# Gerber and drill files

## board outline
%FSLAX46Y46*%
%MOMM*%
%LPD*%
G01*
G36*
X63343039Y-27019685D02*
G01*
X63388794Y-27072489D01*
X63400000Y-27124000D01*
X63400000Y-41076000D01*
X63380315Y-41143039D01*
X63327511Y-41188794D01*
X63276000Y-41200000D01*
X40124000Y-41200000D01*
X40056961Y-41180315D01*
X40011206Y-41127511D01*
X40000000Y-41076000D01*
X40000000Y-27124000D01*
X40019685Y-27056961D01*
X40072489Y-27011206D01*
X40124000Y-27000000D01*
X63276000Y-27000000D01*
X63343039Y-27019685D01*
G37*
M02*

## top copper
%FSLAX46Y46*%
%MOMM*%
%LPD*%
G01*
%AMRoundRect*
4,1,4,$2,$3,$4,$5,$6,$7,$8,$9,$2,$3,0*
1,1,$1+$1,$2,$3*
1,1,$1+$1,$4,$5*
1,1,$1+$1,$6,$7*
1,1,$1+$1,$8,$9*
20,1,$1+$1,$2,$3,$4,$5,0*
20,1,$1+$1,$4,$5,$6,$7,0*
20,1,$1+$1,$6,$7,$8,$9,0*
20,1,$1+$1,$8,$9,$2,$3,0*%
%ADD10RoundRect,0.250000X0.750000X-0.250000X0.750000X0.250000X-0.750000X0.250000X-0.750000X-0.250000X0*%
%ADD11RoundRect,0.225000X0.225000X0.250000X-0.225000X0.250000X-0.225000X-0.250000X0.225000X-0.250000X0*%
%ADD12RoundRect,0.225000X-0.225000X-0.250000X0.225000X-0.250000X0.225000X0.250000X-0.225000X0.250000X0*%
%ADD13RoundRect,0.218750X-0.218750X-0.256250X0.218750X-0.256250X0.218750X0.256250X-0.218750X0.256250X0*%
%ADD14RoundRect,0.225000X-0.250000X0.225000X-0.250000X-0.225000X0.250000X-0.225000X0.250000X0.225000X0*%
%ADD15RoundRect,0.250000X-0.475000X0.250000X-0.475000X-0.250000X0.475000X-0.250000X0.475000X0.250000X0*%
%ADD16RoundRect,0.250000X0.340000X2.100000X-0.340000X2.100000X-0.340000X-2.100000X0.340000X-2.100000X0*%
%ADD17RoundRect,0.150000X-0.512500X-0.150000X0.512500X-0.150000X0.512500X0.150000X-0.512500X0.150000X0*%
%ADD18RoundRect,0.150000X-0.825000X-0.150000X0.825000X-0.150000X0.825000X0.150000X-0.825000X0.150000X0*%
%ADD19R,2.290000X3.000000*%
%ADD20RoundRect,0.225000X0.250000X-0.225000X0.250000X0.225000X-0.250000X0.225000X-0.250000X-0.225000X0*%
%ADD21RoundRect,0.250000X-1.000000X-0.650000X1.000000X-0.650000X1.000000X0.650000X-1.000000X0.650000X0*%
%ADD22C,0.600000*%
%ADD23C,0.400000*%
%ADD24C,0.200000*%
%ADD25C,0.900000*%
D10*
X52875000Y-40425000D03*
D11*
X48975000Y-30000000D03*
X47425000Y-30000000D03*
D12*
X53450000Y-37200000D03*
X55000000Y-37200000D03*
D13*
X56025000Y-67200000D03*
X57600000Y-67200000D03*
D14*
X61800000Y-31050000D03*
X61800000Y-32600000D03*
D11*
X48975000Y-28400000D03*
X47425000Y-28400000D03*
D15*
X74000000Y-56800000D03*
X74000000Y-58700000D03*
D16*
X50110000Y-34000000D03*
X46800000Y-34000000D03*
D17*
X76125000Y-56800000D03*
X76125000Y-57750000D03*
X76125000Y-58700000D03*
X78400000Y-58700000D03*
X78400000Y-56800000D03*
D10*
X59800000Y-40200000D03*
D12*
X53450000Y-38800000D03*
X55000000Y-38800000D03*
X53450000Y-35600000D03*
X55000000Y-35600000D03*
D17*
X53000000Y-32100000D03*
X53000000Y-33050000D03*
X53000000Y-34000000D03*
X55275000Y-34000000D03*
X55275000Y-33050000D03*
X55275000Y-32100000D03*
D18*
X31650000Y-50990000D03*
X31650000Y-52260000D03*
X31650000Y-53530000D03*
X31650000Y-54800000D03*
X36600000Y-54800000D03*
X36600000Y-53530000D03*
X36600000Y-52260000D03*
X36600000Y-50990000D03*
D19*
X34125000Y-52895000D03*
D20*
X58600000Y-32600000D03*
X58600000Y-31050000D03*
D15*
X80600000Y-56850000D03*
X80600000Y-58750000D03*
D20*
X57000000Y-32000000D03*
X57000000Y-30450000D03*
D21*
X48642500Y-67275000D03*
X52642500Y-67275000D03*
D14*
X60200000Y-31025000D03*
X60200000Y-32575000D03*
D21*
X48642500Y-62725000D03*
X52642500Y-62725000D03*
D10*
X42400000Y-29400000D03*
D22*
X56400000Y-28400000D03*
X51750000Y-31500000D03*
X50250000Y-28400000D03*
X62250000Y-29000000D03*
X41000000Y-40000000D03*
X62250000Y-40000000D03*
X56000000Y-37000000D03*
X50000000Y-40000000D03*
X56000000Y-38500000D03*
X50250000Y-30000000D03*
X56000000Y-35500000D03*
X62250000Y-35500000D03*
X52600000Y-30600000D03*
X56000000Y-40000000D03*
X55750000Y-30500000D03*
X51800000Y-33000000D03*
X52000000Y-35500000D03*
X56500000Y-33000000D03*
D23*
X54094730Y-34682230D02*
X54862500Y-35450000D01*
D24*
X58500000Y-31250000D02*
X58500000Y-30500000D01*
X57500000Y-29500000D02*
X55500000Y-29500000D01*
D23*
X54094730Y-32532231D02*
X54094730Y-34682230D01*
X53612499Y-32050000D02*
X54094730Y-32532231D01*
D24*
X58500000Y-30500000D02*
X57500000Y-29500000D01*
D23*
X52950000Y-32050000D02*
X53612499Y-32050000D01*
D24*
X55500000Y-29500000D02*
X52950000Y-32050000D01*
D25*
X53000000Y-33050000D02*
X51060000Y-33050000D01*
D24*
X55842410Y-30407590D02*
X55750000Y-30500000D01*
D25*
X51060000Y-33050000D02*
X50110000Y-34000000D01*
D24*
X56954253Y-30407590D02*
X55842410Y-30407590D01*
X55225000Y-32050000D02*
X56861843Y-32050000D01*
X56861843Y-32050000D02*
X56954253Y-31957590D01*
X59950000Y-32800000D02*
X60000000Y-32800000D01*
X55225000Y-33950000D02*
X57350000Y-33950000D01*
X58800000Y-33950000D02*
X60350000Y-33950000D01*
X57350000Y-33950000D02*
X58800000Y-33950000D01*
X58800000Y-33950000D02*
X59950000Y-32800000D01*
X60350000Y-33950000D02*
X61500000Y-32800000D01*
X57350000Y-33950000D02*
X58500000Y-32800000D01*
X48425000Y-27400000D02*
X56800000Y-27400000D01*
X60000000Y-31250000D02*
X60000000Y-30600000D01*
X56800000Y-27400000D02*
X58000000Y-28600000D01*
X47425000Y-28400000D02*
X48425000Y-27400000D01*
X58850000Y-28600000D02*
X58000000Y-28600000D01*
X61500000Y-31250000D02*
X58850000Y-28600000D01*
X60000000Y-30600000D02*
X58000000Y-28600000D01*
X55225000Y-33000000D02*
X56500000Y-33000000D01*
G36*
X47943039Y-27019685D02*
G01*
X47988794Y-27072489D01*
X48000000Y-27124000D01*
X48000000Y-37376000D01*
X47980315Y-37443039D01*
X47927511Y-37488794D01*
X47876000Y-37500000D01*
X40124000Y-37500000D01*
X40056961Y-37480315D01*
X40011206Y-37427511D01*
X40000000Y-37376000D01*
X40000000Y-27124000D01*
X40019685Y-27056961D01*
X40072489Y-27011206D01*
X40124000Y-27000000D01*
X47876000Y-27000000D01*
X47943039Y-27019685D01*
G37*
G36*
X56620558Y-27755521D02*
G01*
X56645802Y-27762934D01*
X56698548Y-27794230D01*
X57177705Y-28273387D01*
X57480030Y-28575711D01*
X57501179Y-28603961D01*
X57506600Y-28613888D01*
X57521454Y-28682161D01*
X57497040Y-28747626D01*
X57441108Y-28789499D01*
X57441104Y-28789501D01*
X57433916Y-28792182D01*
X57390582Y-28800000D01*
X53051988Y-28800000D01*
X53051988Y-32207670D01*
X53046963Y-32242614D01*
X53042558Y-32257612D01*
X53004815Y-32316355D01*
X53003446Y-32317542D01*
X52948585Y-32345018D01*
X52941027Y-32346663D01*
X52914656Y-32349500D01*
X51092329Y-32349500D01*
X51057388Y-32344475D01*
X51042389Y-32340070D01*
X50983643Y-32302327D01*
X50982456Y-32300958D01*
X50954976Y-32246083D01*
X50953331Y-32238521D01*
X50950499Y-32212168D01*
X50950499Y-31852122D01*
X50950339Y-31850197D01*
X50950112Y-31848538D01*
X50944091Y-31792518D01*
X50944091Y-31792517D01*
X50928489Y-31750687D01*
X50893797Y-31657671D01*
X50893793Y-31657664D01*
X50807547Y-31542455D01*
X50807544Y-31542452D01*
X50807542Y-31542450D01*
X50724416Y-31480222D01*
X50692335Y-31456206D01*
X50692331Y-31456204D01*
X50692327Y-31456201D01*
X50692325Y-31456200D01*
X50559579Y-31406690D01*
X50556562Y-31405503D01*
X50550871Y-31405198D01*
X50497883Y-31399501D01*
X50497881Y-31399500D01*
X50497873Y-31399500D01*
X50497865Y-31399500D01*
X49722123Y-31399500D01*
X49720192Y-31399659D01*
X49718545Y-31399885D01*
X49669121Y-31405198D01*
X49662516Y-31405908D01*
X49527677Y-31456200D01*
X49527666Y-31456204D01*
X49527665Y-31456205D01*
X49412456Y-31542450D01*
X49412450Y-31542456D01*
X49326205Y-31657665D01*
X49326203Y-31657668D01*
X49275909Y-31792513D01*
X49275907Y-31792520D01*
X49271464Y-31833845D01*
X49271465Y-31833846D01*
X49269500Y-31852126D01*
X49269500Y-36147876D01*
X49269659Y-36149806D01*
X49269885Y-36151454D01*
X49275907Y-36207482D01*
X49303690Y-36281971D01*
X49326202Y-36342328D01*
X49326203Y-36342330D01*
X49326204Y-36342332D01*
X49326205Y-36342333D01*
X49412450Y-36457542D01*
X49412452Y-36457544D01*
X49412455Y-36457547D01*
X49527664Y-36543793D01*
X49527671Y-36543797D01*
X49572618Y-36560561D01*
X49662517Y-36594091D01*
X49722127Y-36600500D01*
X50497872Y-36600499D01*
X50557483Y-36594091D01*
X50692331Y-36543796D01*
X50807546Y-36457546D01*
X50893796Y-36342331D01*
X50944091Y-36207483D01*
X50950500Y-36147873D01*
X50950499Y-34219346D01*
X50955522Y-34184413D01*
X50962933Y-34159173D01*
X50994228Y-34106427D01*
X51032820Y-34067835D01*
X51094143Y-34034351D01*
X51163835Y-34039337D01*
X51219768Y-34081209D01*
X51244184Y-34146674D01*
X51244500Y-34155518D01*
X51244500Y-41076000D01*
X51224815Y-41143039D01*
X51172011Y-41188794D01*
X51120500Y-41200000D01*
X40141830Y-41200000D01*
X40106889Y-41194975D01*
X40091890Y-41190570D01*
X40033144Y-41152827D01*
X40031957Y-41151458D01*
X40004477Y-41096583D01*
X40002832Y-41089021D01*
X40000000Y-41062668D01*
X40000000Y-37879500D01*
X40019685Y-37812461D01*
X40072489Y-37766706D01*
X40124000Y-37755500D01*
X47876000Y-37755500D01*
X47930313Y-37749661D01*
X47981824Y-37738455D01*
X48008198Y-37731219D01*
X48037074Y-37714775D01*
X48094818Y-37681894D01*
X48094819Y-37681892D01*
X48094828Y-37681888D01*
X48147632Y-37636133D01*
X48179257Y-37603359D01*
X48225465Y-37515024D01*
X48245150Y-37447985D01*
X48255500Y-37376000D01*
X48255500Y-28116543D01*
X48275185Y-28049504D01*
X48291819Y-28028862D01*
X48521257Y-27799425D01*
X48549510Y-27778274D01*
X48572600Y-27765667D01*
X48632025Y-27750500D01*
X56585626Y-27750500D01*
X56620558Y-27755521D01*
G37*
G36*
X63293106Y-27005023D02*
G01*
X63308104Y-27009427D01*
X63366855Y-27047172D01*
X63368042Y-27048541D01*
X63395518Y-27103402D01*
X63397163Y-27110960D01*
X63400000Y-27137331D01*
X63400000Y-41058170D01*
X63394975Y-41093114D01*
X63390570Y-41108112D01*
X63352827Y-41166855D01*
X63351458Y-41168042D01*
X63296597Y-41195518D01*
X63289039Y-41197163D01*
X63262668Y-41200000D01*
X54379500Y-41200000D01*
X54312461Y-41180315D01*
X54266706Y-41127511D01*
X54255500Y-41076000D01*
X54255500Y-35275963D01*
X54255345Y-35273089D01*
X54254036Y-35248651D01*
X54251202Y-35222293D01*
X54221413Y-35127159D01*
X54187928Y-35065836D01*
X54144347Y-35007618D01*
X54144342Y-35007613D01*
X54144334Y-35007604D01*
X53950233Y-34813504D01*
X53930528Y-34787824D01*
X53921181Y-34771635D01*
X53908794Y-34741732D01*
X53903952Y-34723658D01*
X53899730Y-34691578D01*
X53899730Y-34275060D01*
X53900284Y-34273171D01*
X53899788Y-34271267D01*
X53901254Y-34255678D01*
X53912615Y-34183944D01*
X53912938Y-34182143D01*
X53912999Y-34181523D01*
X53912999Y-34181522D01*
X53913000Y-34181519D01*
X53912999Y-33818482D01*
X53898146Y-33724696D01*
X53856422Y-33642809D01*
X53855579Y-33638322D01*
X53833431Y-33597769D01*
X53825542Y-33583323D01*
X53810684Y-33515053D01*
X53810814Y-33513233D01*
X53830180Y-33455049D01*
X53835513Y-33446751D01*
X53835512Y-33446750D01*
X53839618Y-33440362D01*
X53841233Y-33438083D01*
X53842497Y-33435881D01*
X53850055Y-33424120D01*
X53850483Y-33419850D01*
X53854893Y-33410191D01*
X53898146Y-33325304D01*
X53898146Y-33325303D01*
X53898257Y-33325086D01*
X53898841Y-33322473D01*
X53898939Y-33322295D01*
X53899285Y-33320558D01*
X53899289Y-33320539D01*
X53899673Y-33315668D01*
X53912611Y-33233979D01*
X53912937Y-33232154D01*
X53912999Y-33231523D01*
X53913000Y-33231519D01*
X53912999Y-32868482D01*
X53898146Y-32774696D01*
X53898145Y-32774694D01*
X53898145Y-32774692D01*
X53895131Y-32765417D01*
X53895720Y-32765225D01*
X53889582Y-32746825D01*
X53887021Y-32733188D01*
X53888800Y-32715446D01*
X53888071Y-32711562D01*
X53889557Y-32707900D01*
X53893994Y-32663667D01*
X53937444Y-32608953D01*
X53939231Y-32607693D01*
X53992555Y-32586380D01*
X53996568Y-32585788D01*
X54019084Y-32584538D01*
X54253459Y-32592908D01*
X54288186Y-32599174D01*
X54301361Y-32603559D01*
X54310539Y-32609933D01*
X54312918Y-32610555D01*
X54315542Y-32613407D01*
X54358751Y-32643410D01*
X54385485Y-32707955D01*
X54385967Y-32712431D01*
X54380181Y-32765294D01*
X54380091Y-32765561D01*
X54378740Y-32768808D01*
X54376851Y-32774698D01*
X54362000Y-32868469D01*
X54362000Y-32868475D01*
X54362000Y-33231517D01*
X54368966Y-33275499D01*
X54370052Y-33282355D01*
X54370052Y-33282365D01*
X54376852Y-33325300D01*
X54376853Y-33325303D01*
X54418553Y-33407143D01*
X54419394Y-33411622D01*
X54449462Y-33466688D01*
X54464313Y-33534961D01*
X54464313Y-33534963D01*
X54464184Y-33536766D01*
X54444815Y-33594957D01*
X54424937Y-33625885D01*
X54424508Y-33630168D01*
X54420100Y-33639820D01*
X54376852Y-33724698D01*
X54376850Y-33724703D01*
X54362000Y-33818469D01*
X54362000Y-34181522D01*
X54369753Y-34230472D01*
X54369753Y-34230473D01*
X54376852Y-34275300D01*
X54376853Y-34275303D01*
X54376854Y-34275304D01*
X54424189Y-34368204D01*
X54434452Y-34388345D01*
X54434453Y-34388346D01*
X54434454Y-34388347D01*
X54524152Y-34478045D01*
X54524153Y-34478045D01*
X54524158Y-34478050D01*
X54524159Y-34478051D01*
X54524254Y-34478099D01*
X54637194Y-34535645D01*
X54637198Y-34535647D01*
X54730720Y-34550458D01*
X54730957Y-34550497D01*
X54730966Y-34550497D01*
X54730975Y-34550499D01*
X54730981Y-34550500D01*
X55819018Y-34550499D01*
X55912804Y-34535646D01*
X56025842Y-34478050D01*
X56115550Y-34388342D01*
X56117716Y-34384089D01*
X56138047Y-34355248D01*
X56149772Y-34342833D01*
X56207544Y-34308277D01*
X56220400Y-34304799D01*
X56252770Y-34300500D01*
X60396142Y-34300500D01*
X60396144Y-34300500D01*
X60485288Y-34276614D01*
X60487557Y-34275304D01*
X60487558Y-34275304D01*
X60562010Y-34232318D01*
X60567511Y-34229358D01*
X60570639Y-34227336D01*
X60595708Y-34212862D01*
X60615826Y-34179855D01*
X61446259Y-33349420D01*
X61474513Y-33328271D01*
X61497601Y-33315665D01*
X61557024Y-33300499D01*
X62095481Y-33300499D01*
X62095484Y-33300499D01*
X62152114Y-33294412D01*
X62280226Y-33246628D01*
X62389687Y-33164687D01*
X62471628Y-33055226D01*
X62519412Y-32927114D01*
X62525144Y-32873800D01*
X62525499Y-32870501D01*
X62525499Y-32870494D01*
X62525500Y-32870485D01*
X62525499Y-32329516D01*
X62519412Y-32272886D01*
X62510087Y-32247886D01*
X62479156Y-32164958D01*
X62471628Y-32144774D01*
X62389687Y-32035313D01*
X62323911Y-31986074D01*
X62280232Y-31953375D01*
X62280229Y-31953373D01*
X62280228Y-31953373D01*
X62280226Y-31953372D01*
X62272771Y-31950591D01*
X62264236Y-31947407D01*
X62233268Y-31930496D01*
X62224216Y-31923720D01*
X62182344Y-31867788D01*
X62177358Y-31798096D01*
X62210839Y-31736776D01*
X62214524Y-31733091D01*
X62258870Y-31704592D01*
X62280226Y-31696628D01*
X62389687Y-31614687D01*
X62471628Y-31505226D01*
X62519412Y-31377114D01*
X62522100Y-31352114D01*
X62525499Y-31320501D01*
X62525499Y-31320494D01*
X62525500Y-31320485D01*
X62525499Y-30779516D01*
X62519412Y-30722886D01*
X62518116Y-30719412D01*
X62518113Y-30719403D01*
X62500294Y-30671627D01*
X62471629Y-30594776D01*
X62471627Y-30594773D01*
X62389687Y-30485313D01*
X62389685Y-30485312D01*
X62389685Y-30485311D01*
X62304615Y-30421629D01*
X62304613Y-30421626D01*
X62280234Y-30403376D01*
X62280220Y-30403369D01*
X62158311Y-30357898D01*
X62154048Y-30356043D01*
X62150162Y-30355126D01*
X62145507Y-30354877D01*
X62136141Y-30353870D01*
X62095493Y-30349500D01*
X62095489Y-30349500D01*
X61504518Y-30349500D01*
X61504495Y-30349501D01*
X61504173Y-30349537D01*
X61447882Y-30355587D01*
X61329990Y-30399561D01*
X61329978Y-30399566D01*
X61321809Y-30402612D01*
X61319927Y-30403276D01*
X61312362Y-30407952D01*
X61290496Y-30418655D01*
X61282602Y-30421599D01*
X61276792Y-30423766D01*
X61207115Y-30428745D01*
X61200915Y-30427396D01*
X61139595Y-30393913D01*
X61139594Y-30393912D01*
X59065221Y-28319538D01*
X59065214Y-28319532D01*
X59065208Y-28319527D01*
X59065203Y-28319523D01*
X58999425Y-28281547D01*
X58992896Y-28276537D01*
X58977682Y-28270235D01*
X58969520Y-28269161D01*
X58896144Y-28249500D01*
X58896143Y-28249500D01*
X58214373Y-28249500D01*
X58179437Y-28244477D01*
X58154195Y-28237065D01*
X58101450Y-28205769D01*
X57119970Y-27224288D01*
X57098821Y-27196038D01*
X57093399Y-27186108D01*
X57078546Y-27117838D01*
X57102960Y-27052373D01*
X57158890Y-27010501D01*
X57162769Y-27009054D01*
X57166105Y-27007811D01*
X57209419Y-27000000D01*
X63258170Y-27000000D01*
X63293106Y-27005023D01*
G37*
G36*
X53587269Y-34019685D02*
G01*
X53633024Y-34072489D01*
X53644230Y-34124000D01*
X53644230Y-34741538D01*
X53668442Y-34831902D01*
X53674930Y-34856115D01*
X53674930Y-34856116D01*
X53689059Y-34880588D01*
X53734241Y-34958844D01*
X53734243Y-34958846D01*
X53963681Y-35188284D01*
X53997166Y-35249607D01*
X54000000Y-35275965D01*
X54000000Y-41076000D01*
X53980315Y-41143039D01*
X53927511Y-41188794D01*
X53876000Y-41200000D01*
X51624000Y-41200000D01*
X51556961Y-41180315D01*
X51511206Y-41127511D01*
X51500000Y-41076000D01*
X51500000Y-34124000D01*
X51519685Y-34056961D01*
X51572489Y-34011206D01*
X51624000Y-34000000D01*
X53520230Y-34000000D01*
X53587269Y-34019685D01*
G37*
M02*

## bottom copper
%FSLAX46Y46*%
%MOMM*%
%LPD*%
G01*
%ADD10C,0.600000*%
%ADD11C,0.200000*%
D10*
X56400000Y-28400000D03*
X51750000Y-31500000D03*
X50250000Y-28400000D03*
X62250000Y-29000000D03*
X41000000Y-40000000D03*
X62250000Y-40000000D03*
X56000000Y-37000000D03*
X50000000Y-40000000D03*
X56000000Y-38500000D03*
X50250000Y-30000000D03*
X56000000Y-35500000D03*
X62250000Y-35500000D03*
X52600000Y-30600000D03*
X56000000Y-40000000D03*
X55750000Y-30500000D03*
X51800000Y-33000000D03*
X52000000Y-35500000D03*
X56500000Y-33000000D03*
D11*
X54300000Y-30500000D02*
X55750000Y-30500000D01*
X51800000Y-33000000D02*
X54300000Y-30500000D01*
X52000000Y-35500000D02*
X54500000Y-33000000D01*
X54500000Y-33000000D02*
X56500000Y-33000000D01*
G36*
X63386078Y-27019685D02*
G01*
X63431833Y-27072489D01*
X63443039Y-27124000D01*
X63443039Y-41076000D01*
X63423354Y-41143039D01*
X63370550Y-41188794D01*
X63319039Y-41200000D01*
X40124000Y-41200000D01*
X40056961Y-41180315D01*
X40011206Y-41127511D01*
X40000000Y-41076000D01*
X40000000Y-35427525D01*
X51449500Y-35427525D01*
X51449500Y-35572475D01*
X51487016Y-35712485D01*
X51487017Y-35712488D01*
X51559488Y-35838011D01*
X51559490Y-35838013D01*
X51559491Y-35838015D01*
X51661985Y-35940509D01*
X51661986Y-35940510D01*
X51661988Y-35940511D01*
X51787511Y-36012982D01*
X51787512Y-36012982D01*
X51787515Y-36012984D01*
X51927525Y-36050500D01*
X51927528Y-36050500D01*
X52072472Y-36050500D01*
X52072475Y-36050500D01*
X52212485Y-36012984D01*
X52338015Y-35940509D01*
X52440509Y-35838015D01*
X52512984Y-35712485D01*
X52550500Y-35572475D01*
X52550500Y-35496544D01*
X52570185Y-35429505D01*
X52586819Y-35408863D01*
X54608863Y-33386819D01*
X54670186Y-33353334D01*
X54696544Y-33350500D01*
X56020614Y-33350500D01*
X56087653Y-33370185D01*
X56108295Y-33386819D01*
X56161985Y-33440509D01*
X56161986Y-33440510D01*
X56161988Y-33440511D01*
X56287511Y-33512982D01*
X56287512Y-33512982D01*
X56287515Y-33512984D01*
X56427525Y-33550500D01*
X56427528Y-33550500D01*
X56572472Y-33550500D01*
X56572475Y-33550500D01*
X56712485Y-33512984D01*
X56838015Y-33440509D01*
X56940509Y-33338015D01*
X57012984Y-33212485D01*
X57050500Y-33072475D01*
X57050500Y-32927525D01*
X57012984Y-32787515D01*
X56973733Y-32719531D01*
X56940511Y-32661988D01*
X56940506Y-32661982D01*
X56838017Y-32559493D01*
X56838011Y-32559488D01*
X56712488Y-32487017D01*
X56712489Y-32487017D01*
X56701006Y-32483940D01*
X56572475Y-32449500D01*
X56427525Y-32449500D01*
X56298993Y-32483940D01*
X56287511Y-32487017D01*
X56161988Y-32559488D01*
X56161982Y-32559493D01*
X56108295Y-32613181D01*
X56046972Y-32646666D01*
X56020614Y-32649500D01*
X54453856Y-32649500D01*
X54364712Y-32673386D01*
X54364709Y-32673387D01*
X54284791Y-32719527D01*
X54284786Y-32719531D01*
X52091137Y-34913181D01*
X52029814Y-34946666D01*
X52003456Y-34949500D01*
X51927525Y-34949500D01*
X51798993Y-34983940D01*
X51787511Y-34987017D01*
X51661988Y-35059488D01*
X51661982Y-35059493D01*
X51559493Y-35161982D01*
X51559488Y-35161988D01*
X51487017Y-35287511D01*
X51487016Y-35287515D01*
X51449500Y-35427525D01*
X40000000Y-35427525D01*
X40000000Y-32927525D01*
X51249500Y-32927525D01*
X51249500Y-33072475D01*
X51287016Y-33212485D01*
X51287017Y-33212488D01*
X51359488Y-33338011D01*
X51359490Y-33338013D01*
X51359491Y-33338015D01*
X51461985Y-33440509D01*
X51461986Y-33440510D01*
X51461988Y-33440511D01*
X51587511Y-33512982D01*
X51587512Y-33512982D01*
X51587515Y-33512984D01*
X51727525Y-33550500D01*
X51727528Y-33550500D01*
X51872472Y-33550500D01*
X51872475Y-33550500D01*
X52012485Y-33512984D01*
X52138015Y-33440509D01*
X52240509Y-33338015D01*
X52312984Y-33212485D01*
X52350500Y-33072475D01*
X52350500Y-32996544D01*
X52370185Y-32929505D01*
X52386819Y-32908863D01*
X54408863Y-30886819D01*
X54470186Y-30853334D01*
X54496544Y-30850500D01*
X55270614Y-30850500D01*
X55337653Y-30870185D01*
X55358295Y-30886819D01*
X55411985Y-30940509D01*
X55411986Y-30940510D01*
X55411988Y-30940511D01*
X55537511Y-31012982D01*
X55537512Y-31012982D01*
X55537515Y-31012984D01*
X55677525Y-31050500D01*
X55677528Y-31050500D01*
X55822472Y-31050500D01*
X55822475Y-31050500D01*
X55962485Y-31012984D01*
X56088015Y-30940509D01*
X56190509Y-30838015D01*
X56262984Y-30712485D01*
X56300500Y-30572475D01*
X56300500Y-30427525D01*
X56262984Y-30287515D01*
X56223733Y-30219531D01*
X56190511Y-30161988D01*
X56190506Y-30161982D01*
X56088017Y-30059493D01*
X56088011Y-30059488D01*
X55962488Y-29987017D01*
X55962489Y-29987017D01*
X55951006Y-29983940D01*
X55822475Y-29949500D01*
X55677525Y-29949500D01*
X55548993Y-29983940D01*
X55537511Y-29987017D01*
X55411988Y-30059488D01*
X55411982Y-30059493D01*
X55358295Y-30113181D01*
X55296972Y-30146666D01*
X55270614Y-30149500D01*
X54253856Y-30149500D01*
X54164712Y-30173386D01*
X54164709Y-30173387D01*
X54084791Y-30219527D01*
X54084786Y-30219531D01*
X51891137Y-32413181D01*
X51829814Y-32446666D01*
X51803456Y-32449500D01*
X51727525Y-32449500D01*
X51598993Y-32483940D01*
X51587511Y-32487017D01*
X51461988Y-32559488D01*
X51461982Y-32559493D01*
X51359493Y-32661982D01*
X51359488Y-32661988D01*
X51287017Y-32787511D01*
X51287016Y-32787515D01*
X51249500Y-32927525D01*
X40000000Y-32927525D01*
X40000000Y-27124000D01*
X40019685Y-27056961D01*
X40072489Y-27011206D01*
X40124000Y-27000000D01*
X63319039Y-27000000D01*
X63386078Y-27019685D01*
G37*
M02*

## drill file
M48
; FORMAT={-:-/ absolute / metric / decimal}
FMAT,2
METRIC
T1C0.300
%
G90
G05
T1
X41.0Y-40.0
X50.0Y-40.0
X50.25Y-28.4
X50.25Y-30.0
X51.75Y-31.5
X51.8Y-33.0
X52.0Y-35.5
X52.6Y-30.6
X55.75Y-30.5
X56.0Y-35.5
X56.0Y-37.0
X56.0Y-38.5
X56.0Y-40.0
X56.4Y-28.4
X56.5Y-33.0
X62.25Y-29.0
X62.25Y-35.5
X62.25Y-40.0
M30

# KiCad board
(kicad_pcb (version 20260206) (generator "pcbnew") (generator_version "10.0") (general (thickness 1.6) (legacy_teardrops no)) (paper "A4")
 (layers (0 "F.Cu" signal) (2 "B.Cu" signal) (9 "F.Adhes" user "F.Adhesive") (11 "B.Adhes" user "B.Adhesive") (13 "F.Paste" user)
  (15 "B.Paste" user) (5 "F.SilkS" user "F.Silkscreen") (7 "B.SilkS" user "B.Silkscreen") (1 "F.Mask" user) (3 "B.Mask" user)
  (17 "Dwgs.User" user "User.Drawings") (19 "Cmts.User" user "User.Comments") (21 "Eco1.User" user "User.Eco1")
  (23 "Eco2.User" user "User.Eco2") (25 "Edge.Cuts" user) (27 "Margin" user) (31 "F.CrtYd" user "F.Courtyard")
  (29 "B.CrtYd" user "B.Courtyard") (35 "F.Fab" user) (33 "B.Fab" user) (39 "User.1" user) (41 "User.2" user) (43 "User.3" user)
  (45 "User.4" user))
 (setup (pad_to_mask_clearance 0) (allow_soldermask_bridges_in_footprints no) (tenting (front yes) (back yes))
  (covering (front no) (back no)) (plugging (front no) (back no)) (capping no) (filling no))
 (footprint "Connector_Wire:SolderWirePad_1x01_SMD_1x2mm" (layer "F.Cu") (at 52.875 40.425 90)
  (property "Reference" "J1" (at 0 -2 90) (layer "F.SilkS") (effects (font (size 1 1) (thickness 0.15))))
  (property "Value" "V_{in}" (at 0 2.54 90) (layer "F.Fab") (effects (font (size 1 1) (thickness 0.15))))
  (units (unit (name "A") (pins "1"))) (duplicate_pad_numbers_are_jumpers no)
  (pad "1" smd roundrect (at 0 0 90) (size 1 2) (layers "F.Cu" "F.Mask") (roundrect_rratio 0.25) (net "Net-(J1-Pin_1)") (zone_connect 2)))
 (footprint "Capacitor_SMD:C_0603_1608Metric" (layer "F.Cu") (at 48.2 30 180)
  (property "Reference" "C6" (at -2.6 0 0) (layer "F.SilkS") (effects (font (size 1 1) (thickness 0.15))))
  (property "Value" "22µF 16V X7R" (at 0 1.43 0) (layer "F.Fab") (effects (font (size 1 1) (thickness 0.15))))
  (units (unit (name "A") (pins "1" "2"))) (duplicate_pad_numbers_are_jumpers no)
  (pad "1" smd roundrect (at -0.775 0 180) (size 0.9 0.95) (layers "F.Cu" "F.Mask" "F.Paste") (roundrect_rratio 0.25) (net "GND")
   (zone_connect 2))
  (pad "2" smd roundrect (at 0.775 0 180) (size 0.9 0.95) (layers "F.Cu" "F.Mask" "F.Paste") (roundrect_rratio 0.25) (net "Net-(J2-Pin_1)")
   (zone_connect 2)))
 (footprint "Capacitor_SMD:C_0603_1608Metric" (layer "F.Cu") (at 54.225 37.2)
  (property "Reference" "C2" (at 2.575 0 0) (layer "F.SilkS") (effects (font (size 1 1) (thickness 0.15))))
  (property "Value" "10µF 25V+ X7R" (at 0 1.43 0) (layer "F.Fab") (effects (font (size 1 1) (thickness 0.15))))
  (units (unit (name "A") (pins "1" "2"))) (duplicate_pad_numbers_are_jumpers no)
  (pad "1" smd roundrect (at -0.775 0) (size 0.9 0.95) (layers "F.Cu" "F.Mask" "F.Paste") (roundrect_rratio 0.25) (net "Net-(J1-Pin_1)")
   (zone_connect 2))
  (pad "2" smd roundrect (at 0.775 0) (size 0.9 0.95) (layers "F.Cu" "F.Mask" "F.Paste") (roundrect_rratio 0.25) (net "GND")
   (zone_connect 2)))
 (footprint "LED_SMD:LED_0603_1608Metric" (layer "F.Cu") (at 56.8125 67.2)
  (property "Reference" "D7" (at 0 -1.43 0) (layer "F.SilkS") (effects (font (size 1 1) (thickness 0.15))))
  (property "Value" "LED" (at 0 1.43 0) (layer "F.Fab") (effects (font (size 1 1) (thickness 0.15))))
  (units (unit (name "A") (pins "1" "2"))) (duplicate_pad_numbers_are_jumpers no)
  (pad "1" smd roundrect (at -0.7875 0) (size 0.875 0.95) (layers "F.Cu" "F.Mask" "F.Paste") (roundrect_rratio 0.25) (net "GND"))
  (pad "2" smd roundrect (at 0.7875 0) (size 0.875 0.95) (layers "F.Cu" "F.Mask" "F.Paste") (roundrect_rratio 0.25) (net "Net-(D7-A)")))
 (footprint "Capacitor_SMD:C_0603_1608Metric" (layer "F.Cu") (at 61.8 31.825 -90)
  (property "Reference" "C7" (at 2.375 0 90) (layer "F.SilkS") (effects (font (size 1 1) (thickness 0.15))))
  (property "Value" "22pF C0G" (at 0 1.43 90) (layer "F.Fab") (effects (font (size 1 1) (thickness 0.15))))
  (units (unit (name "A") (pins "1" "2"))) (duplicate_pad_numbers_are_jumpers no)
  (pad "1" smd roundrect (at -0.775 0 270) (size 0.9 0.95) (layers "F.Cu" "F.Mask" "F.Paste") (roundrect_rratio 0.25) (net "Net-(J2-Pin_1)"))
  (pad "2" smd roundrect (at 0.775 0 270) (size 0.9 0.95) (layers "F.Cu" "F.Mask" "F.Paste") (roundrect_rratio 0.25) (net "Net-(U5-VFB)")))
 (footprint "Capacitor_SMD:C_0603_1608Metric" (layer "F.Cu") (at 48.2 28.4 180)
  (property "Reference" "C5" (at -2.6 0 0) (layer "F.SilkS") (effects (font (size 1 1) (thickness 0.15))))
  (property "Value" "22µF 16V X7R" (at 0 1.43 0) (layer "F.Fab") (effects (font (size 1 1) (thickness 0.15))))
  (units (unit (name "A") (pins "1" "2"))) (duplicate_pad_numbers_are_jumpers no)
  (pad "1" smd roundrect (at -0.775 0 180) (size 0.9 0.95) (layers "F.Cu" "F.Mask" "F.Paste") (roundrect_rratio 0.25) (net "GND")
   (zone_connect 2))
  (pad "2" smd roundrect (at 0.775 0 180) (size 0.9 0.95) (layers "F.Cu" "F.Mask" "F.Paste") (roundrect_rratio 0.25) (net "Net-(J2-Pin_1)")
   (zone_connect 2)))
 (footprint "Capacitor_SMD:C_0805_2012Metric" (layer "F.Cu") (at 74 57.75 -90)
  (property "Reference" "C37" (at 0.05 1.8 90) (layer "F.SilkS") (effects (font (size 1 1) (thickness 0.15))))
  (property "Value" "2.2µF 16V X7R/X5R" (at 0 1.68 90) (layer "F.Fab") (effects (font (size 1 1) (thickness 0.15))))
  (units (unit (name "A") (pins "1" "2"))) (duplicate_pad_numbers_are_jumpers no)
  (pad "1" smd roundrect (at -0.95 0 270) (size 1 1.45) (layers "F.Cu" "F.Mask" "F.Paste") (roundrect_rratio 0.25) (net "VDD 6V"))
  (pad "2" smd roundrect (at 0.95 0 270) (size 1 1.45) (layers "F.Cu" "F.Mask" "F.Paste") (roundrect_rratio 0.25) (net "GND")))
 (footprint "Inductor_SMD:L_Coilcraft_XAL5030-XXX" (layer "F.Cu") (at 48.455 34 180)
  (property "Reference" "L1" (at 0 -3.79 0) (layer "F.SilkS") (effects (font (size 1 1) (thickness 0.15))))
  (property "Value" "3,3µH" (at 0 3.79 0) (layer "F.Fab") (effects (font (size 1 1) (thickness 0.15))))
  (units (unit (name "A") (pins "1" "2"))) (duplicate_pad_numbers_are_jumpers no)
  (pad "1" smd roundrect (at -1.655 0 180) (size 1.18 4.7) (layers "F.Cu" "F.Mask" "F.Paste") (roundrect_rratio 0.211864)
   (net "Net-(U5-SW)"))
  (pad "2" smd roundrect (at 1.655 0 180) (size 1.18 4.7) (layers "F.Cu" "F.Mask" "F.Paste") (roundrect_rratio 0.211864)
   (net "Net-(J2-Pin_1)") (zone_connect 2)))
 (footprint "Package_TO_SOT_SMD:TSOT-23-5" (layer "F.Cu") (at 77.2625 57.75)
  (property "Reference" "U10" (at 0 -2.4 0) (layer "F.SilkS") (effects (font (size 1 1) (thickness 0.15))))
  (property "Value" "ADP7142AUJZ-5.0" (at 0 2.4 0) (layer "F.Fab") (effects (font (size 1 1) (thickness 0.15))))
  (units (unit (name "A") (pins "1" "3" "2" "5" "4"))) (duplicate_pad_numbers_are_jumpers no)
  (pad "1" smd roundrect (at -1.1375 -0.95) (size 1.325 0.6) (layers "F.Cu" "F.Mask" "F.Paste") (roundrect_rratio 0.25) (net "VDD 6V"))
  (pad "2" smd roundrect (at -1.1375 0) (size 1.325 0.6) (layers "F.Cu" "F.Mask" "F.Paste") (roundrect_rratio 0.25) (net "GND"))
  (pad "3" smd roundrect (at -1.1375 0.95) (size 1.325 0.6) (layers "F.Cu" "F.Mask" "F.Paste") (roundrect_rratio 0.25) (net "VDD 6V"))
  (pad "4" smd roundrect (at 1.1375 0.95) (size 1.325 0.6) (layers "F.Cu" "F.Mask" "F.Paste") (roundrect_rratio 0.25) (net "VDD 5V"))
  (pad "5" smd roundrect (at 1.1375 -0.95) (size 1.325 0.6) (layers "F.Cu" "F.Mask" "F.Paste") (roundrect_rratio 0.25) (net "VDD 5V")))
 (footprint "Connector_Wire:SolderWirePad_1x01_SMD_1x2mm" (layer "F.Cu") (at 59.8 40.2 90)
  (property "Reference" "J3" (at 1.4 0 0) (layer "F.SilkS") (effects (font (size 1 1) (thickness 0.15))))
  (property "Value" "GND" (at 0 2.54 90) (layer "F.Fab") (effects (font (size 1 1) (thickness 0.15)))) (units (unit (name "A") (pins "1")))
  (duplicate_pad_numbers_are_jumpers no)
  (pad "1" smd roundrect (at 0 0 90) (size 1 2) (layers "F.Cu" "F.Mask") (roundrect_rratio 0.25) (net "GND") (zone_connect 2)))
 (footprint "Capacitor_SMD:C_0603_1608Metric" (layer "F.Cu") (at 54.225 38.8)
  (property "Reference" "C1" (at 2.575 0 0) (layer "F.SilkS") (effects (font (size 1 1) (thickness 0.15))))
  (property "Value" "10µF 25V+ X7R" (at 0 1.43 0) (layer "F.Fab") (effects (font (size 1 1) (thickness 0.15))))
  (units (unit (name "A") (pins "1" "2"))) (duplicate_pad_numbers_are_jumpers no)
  (pad "1" smd roundrect (at -0.775 0) (size 0.9 0.95) (layers "F.Cu" "F.Mask" "F.Paste") (roundrect_rratio 0.25) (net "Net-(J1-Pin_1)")
   (zone_connect 2))
  (pad "2" smd roundrect (at 0.775 0) (size 0.9 0.95) (layers "F.Cu" "F.Mask" "F.Paste") (roundrect_rratio 0.25) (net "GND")
   (zone_connect 2)))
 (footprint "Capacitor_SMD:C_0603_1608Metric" (layer "F.Cu") (at 54.225 35.6)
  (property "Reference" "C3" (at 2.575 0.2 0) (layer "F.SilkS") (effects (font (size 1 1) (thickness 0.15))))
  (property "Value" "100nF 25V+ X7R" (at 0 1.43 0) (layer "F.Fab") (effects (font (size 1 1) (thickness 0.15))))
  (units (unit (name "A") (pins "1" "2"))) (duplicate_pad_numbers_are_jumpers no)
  (pad "1" smd roundrect (at -0.775 0) (size 0.9 0.95) (layers "F.Cu" "F.Mask" "F.Paste") (roundrect_rratio 0.25) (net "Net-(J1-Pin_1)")
   (zone_connect 2))
  (pad "2" smd roundrect (at 0.775 0) (size 0.9 0.95) (layers "F.Cu" "F.Mask" "F.Paste") (roundrect_rratio 0.25) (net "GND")
   (zone_connect 2)))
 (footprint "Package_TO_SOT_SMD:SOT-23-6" (layer "F.Cu") (at 54.1375 33.05)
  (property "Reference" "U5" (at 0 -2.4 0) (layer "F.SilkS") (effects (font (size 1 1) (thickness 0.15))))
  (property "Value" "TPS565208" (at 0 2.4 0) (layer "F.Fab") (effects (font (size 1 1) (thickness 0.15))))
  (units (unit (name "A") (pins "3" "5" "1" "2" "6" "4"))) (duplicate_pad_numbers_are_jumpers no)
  (pad "1" smd roundrect (at -1.1375 -0.95) (size 1.325 0.6) (layers "F.Cu" "F.Mask" "F.Paste") (roundrect_rratio 0.25) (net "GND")
   (zone_connect 2))
  (pad "2" smd roundrect (at -1.1375 0) (size 1.325 0.6) (layers "F.Cu" "F.Mask" "F.Paste") (roundrect_rratio 0.25) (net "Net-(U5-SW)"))
  (pad "3" smd roundrect (at -1.1375 0.95) (size 1.325 0.6) (layers "F.Cu" "F.Mask" "F.Paste") (roundrect_rratio 0.25)
   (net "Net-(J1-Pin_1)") (zone_connect 2))
  (pad "4" smd roundrect (at 1.1375 0.95) (size 1.325 0.6) (layers "F.Cu" "F.Mask" "F.Paste") (roundrect_rratio 0.25) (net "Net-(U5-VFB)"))
  (pad "5" smd roundrect (at 1.1375 0) (size 1.325 0.6) (layers "F.Cu" "F.Mask" "F.Paste") (roundrect_rratio 0.25) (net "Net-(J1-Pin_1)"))
  (pad "6" smd roundrect (at 1.1375 -0.95) (size 1.325 0.6) (layers "F.Cu" "F.Mask" "F.Paste") (roundrect_rratio 0.25) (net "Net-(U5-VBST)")))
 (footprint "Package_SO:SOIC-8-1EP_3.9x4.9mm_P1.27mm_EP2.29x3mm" (layer "F.Cu") (at 34.125 52.895)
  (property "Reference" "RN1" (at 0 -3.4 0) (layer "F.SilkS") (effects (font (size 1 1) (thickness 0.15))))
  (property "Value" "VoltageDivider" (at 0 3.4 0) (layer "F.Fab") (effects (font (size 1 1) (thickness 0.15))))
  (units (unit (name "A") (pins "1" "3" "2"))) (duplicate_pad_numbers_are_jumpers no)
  (pad "" smd roundrect (at -0.57 -0.75) (size 0.92 1.21) (layers "F.Paste") (roundrect_rratio 0.25))
  (pad "" smd roundrect (at -0.57 0.75) (size 0.92 1.21) (layers "F.Paste") (roundrect_rratio 0.25))
  (pad "" smd roundrect (at 0.57 -0.75) (size 0.92 1.21) (layers "F.Paste") (roundrect_rratio 0.25))
  (pad "" smd roundrect (at 0.57 0.75) (size 0.92 1.21) (layers "F.Paste") (roundrect_rratio 0.25))
  (pad "1" smd roundrect (at -2.475 -1.905) (size 1.95 0.6) (layers "F.Cu" "F.Mask" "F.Paste") (roundrect_rratio 0.25) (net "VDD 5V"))
  (pad "2" smd roundrect (at -2.475 -0.635) (size 1.95 0.6) (layers "F.Cu" "F.Mask" "F.Paste") (roundrect_rratio 0.25) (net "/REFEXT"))
  (pad "3" smd roundrect (at -2.475 0.635) (size 1.95 0.6) (layers "F.Cu" "F.Mask" "F.Paste") (roundrect_rratio 0.25) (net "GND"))
  (pad "4" smd roundrect (at -2.475 1.905) (size 1.95 0.6) (layers "F.Cu" "F.Mask" "F.Paste") (roundrect_rratio 0.25))
  (pad "5" smd roundrect (at 2.475 1.905) (size 1.95 0.6) (layers "F.Cu" "F.Mask" "F.Paste") (roundrect_rratio 0.25))
  (pad "6" smd roundrect (at 2.475 0.635) (size 1.95 0.6) (layers "F.Cu" "F.Mask" "F.Paste") (roundrect_rratio 0.25))
  (pad "7" smd roundrect (at 2.475 -0.635) (size 1.95 0.6) (layers "F.Cu" "F.Mask" "F.Paste") (roundrect_rratio 0.25))
  (pad "8" smd roundrect (at 2.475 -1.905) (size 1.95 0.6) (layers "F.Cu" "F.Mask" "F.Paste") (roundrect_rratio 0.25))
  (pad "9" smd rect (at 0 0) (size 2.29 3) (layers "F.Cu" "F.Mask") (zone_connect 2)))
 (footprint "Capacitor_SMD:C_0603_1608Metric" (layer "F.Cu") (at 58.6 31.825 90)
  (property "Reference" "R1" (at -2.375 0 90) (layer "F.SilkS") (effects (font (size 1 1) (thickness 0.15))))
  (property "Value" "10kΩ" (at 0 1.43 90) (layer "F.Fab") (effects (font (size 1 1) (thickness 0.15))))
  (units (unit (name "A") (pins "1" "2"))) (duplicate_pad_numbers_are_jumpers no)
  (pad "1" smd roundrect (at -0.775 0 90) (size 0.9 0.95) (layers "F.Cu" "F.Mask" "F.Paste") (roundrect_rratio 0.25) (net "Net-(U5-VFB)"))
  (pad "2" smd roundrect (at 0.775 0 90) (size 0.9 0.95) (layers "F.Cu" "F.Mask" "F.Paste") (roundrect_rratio 0.25) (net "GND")))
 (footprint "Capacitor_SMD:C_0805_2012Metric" (layer "F.Cu") (at 80.6 57.8 -90)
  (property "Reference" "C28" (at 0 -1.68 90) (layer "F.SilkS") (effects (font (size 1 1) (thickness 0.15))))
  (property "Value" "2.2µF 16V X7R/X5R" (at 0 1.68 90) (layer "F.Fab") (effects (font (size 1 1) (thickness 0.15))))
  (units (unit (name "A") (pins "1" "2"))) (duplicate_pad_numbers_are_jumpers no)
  (pad "1" smd roundrect (at -0.95 0 270) (size 1 1.45) (layers "F.Cu" "F.Mask" "F.Paste") (roundrect_rratio 0.25) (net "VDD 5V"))
  (pad "2" smd roundrect (at 0.95 0 270) (size 1 1.45) (layers "F.Cu" "F.Mask" "F.Paste") (roundrect_rratio 0.25) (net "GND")))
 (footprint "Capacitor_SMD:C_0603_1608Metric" (layer "F.Cu") (at 57 31.225 90)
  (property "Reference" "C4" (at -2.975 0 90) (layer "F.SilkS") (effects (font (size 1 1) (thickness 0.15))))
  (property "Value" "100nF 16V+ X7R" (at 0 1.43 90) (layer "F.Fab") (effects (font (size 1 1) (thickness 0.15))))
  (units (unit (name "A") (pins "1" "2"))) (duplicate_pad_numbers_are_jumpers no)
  (pad "1" smd roundrect (at -0.775 0 90) (size 0.9 0.95) (layers "F.Cu" "F.Mask" "F.Paste") (roundrect_rratio 0.25) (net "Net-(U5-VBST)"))
  (pad "2" smd roundrect (at 0.775 0 90) (size 0.9 0.95) (layers "F.Cu" "F.Mask" "F.Paste") (roundrect_rratio 0.25) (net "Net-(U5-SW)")))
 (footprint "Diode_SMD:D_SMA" (layer "F.Cu") (at 50.6425 67.275)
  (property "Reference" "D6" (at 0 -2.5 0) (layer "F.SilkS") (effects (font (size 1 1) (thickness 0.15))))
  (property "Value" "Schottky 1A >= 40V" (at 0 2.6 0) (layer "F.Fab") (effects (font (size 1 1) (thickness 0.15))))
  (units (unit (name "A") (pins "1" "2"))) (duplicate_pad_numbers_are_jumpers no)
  (pad "1" smd roundrect (at -2 0) (size 2.5 1.8) (layers "F.Cu" "F.Mask" "F.Paste") (roundrect_rratio 0.1388888889) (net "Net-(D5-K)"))
  (pad "2" smd roundrect (at 2 0) (size 2.5 1.8) (layers "F.Cu" "F.Mask" "F.Paste") (roundrect_rratio 0.1388888889) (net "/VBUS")))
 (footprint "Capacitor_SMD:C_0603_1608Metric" (layer "F.Cu") (at 60.2 31.8 -90)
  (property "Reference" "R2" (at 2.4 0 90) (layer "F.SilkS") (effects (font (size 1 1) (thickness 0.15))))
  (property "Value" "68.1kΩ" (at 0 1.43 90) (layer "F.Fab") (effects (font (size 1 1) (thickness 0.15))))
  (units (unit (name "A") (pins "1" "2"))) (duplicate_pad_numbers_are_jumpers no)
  (pad "1" smd roundrect (at -0.775 0 270) (size 0.9 0.95) (layers "F.Cu" "F.Mask" "F.Paste") (roundrect_rratio 0.25) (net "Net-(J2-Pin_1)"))
  (pad "2" smd roundrect (at 0.775 0 270) (size 0.9 0.95) (layers "F.Cu" "F.Mask" "F.Paste") (roundrect_rratio 0.25) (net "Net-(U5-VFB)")))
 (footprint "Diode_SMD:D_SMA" (layer "F.Cu") (at 50.6425 62.725)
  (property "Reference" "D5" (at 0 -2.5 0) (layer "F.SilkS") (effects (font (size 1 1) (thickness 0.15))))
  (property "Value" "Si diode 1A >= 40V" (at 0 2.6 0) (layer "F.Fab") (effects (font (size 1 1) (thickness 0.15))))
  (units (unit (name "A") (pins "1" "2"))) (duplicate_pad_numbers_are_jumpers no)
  (pad "1" smd roundrect (at -2 0) (size 2.5 1.8) (layers "F.Cu" "F.Mask" "F.Paste") (roundrect_rratio 0.1388888889) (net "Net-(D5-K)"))
  (pad "2" smd roundrect (at 2 0) (size 2.5 1.8) (layers "F.Cu" "F.Mask" "F.Paste") (roundrect_rratio 0.1388888889) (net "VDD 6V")))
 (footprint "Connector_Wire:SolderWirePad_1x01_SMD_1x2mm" (layer "F.Cu") (at 42.4 29.4 90)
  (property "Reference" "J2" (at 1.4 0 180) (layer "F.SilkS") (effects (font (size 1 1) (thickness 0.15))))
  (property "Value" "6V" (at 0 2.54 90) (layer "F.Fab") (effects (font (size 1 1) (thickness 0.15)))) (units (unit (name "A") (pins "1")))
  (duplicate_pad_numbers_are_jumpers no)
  (pad "1" smd roundrect (at 0 0 90) (size 1 2) (layers "F.Cu" "F.Mask") (roundrect_rratio 0.25) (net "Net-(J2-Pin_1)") (zone_connect 2)))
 (segment (start 54.09473 34.68223) (end 54.8625 35.45) (width 0.4) (layer "F.Cu") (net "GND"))
 (segment (start 58.5 31.25) (end 58.5 30.5) (width 0.2) (layer "F.Cu") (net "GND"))
 (segment (start 57.5 29.5) (end 55.5 29.5) (width 0.2) (layer "F.Cu") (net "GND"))
 (segment (start 54.09473 32.532231) (end 54.09473 34.68223) (width 0.4) (layer "F.Cu") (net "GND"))
 (segment (start 53.612499 32.05) (end 54.09473 32.532231) (width 0.4) (layer "F.Cu") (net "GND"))
 (segment (start 58.5 30.5) (end 57.5 29.5) (width 0.2) (layer "F.Cu") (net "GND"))
 (segment (start 52.95 32.05) (end 53.612499 32.05) (width 0.4) (layer "F.Cu") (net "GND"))
 (segment (start 55.5 29.5) (end 52.95 32.05) (width 0.2) (layer "F.Cu") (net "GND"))
 (via (at 56.4 28.4) (size 0.6) (drill 0.3) (layers "F.Cu" "B.Cu") (free yes) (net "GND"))
 (via (at 51.75 31.5) (size 0.6) (drill 0.3) (layers "F.Cu" "B.Cu") (free yes) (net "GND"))
 (via (at 50.25 28.4) (size 0.6) (drill 0.3) (layers "F.Cu" "B.Cu") (free yes) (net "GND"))
 (via (at 62.25 29) (size 0.6) (drill 0.3) (layers "F.Cu" "B.Cu") (free yes) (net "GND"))
 (via (at 41 40) (size 0.6) (drill 0.3) (layers "F.Cu" "B.Cu") (free yes) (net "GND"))
 (via (at 62.25 40) (size 0.6) (drill 0.3) (layers "F.Cu" "B.Cu") (free yes) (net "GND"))
 (via (at 56 37) (size 0.6) (drill 0.3) (layers "F.Cu" "B.Cu") (free yes) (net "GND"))
 (via (at 50 40) (size 0.6) (drill 0.3) (layers "F.Cu" "B.Cu") (free yes) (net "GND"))
 (via (at 56 38.5) (size 0.6) (drill 0.3) (layers "F.Cu" "B.Cu") (free yes) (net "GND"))
 (via (at 50.25 30) (size 0.6) (drill 0.3) (layers "F.Cu" "B.Cu") (free yes) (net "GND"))
 (via (at 56 35.5) (size 0.6) (drill 0.3) (layers "F.Cu" "B.Cu") (free yes) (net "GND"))
 (via (at 62.25 35.5) (size 0.6) (drill 0.3) (layers "F.Cu" "B.Cu") (free yes) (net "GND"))
 (via (at 52.6 30.6) (size 0.6) (drill 0.3) (layers "F.Cu" "B.Cu") (free yes) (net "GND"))
 (via (at 56 40) (size 0.6) (drill 0.3) (layers "F.Cu" "B.Cu") (free yes) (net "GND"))
 (segment (start 53 33.05) (end 51.06 33.05) (width 0.9) (layer "F.Cu") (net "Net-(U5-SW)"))
 (segment (start 55.84241 30.40759) (end 55.75 30.5) (width 0.2) (layer "F.Cu") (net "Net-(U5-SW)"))
 (segment (start 51.06 33.05) (end 50.11 34) (width 0.9) (layer "F.Cu") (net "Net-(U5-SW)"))
 (segment (start 56.954253 30.40759) (end 55.84241 30.40759) (width 0.2) (layer "F.Cu") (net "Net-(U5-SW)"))
 (via (at 55.75 30.5) (size 0.6) (drill 0.3) (layers "F.Cu" "B.Cu") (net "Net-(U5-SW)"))
 (via (at 51.8 33) (size 0.6) (drill 0.3) (layers "F.Cu" "B.Cu") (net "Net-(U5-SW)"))
 (segment (start 54.3 30.5) (end 55.75 30.5) (width 0.2) (layer "B.Cu") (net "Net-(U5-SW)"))
 (segment (start 51.8 33) (end 54.3 30.5) (width 0.2) (layer "B.Cu") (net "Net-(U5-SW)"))
 (segment (start 55.225 32.05) (end 56.861843 32.05) (width 0.2) (layer "F.Cu") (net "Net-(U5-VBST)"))
 (segment (start 56.861843 32.05) (end 56.954253 31.95759) (width 0.2) (layer "F.Cu") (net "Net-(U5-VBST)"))
 (segment (start 59.95 32.8) (end 60 32.8) (width 0.2) (layer "F.Cu") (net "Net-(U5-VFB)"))
 (segment (start 55.225 33.95) (end 57.35 33.95) (width 0.2) (layer "F.Cu") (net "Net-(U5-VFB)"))
 (segment (start 58.8 33.95) (end 60.35 33.95) (width 0.2) (layer "F.Cu") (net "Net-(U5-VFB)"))
 (segment (start 57.35 33.95) (end 58.8 33.95) (width 0.2) (layer "F.Cu") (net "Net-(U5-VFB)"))
 (segment (start 58.8 33.95) (end 59.95 32.8) (width 0.2) (layer "F.Cu") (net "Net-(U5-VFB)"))
 (segment (start 60.35 33.95) (end 61.5 32.8) (width 0.2) (layer "F.Cu") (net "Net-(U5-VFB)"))
 (segment (start 57.35 33.95) (end 58.5 32.8) (width 0.2) (layer "F.Cu") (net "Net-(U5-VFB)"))
 (segment (start 48.425 27.4) (end 56.8 27.4) (width 0.2) (layer "F.Cu") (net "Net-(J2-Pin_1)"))
 (segment (start 60 31.25) (end 60 30.6) (width 0.2) (layer "F.Cu") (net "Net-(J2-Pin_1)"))
 (segment (start 56.8 27.4) (end 58 28.6) (width 0.2) (layer "F.Cu") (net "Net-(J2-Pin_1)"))
 (segment (start 47.425 28.4) (end 48.425 27.4) (width 0.2) (layer "F.Cu") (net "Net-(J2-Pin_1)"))
 (segment (start 58.85 28.6) (end 58 28.6) (width 0.2) (layer "F.Cu") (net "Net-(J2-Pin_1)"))
 (segment (start 61.5 31.25) (end 58.85 28.6) (width 0.2) (layer "F.Cu") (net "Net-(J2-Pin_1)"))
 (segment (start 60 30.6) (end 58 28.6) (width 0.2) (layer "F.Cu") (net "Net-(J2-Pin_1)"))
 (segment (start 55.225 33) (end 56.5 33) (width 0.2) (layer "F.Cu") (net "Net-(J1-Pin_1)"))
 (via (at 52 35.5) (size 0.6) (drill 0.3) (layers "F.Cu" "B.Cu") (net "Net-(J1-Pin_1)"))
 (via (at 56.5 33) (size 0.6) (drill 0.3) (layers "F.Cu" "B.Cu") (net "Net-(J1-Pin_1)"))
 (segment (start 52 35.5) (end 54.5 33) (width 0.2) (layer "B.Cu") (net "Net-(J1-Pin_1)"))
 (segment (start 54.5 33) (end 56.5 33) (width 0.2) (layer "B.Cu") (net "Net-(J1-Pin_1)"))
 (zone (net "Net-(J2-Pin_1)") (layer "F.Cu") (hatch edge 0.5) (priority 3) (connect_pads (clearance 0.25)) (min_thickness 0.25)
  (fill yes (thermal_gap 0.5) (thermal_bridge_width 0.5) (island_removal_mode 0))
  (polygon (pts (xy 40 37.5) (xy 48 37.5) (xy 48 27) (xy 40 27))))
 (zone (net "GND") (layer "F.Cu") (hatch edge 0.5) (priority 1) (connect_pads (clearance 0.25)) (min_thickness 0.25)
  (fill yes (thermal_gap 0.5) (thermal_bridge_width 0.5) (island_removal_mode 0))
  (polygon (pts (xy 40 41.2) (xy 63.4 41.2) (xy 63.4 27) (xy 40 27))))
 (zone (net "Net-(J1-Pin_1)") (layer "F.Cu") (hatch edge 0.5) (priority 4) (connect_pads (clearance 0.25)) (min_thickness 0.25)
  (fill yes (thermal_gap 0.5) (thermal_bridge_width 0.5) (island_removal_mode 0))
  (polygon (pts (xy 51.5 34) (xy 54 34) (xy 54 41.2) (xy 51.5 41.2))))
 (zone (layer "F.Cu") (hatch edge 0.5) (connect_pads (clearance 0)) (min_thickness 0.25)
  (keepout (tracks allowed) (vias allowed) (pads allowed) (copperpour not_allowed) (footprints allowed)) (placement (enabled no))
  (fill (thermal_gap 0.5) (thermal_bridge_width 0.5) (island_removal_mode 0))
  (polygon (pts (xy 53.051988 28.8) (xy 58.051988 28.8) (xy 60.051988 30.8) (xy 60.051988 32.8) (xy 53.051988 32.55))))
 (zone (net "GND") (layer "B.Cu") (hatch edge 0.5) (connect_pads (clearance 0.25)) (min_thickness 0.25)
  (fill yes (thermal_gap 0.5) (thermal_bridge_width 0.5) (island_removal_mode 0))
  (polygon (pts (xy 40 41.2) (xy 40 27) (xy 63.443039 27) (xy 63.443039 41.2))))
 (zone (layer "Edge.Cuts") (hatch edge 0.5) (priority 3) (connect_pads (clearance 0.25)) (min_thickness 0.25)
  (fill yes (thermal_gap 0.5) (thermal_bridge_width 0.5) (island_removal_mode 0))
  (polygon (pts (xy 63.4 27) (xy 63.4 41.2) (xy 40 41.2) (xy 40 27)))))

